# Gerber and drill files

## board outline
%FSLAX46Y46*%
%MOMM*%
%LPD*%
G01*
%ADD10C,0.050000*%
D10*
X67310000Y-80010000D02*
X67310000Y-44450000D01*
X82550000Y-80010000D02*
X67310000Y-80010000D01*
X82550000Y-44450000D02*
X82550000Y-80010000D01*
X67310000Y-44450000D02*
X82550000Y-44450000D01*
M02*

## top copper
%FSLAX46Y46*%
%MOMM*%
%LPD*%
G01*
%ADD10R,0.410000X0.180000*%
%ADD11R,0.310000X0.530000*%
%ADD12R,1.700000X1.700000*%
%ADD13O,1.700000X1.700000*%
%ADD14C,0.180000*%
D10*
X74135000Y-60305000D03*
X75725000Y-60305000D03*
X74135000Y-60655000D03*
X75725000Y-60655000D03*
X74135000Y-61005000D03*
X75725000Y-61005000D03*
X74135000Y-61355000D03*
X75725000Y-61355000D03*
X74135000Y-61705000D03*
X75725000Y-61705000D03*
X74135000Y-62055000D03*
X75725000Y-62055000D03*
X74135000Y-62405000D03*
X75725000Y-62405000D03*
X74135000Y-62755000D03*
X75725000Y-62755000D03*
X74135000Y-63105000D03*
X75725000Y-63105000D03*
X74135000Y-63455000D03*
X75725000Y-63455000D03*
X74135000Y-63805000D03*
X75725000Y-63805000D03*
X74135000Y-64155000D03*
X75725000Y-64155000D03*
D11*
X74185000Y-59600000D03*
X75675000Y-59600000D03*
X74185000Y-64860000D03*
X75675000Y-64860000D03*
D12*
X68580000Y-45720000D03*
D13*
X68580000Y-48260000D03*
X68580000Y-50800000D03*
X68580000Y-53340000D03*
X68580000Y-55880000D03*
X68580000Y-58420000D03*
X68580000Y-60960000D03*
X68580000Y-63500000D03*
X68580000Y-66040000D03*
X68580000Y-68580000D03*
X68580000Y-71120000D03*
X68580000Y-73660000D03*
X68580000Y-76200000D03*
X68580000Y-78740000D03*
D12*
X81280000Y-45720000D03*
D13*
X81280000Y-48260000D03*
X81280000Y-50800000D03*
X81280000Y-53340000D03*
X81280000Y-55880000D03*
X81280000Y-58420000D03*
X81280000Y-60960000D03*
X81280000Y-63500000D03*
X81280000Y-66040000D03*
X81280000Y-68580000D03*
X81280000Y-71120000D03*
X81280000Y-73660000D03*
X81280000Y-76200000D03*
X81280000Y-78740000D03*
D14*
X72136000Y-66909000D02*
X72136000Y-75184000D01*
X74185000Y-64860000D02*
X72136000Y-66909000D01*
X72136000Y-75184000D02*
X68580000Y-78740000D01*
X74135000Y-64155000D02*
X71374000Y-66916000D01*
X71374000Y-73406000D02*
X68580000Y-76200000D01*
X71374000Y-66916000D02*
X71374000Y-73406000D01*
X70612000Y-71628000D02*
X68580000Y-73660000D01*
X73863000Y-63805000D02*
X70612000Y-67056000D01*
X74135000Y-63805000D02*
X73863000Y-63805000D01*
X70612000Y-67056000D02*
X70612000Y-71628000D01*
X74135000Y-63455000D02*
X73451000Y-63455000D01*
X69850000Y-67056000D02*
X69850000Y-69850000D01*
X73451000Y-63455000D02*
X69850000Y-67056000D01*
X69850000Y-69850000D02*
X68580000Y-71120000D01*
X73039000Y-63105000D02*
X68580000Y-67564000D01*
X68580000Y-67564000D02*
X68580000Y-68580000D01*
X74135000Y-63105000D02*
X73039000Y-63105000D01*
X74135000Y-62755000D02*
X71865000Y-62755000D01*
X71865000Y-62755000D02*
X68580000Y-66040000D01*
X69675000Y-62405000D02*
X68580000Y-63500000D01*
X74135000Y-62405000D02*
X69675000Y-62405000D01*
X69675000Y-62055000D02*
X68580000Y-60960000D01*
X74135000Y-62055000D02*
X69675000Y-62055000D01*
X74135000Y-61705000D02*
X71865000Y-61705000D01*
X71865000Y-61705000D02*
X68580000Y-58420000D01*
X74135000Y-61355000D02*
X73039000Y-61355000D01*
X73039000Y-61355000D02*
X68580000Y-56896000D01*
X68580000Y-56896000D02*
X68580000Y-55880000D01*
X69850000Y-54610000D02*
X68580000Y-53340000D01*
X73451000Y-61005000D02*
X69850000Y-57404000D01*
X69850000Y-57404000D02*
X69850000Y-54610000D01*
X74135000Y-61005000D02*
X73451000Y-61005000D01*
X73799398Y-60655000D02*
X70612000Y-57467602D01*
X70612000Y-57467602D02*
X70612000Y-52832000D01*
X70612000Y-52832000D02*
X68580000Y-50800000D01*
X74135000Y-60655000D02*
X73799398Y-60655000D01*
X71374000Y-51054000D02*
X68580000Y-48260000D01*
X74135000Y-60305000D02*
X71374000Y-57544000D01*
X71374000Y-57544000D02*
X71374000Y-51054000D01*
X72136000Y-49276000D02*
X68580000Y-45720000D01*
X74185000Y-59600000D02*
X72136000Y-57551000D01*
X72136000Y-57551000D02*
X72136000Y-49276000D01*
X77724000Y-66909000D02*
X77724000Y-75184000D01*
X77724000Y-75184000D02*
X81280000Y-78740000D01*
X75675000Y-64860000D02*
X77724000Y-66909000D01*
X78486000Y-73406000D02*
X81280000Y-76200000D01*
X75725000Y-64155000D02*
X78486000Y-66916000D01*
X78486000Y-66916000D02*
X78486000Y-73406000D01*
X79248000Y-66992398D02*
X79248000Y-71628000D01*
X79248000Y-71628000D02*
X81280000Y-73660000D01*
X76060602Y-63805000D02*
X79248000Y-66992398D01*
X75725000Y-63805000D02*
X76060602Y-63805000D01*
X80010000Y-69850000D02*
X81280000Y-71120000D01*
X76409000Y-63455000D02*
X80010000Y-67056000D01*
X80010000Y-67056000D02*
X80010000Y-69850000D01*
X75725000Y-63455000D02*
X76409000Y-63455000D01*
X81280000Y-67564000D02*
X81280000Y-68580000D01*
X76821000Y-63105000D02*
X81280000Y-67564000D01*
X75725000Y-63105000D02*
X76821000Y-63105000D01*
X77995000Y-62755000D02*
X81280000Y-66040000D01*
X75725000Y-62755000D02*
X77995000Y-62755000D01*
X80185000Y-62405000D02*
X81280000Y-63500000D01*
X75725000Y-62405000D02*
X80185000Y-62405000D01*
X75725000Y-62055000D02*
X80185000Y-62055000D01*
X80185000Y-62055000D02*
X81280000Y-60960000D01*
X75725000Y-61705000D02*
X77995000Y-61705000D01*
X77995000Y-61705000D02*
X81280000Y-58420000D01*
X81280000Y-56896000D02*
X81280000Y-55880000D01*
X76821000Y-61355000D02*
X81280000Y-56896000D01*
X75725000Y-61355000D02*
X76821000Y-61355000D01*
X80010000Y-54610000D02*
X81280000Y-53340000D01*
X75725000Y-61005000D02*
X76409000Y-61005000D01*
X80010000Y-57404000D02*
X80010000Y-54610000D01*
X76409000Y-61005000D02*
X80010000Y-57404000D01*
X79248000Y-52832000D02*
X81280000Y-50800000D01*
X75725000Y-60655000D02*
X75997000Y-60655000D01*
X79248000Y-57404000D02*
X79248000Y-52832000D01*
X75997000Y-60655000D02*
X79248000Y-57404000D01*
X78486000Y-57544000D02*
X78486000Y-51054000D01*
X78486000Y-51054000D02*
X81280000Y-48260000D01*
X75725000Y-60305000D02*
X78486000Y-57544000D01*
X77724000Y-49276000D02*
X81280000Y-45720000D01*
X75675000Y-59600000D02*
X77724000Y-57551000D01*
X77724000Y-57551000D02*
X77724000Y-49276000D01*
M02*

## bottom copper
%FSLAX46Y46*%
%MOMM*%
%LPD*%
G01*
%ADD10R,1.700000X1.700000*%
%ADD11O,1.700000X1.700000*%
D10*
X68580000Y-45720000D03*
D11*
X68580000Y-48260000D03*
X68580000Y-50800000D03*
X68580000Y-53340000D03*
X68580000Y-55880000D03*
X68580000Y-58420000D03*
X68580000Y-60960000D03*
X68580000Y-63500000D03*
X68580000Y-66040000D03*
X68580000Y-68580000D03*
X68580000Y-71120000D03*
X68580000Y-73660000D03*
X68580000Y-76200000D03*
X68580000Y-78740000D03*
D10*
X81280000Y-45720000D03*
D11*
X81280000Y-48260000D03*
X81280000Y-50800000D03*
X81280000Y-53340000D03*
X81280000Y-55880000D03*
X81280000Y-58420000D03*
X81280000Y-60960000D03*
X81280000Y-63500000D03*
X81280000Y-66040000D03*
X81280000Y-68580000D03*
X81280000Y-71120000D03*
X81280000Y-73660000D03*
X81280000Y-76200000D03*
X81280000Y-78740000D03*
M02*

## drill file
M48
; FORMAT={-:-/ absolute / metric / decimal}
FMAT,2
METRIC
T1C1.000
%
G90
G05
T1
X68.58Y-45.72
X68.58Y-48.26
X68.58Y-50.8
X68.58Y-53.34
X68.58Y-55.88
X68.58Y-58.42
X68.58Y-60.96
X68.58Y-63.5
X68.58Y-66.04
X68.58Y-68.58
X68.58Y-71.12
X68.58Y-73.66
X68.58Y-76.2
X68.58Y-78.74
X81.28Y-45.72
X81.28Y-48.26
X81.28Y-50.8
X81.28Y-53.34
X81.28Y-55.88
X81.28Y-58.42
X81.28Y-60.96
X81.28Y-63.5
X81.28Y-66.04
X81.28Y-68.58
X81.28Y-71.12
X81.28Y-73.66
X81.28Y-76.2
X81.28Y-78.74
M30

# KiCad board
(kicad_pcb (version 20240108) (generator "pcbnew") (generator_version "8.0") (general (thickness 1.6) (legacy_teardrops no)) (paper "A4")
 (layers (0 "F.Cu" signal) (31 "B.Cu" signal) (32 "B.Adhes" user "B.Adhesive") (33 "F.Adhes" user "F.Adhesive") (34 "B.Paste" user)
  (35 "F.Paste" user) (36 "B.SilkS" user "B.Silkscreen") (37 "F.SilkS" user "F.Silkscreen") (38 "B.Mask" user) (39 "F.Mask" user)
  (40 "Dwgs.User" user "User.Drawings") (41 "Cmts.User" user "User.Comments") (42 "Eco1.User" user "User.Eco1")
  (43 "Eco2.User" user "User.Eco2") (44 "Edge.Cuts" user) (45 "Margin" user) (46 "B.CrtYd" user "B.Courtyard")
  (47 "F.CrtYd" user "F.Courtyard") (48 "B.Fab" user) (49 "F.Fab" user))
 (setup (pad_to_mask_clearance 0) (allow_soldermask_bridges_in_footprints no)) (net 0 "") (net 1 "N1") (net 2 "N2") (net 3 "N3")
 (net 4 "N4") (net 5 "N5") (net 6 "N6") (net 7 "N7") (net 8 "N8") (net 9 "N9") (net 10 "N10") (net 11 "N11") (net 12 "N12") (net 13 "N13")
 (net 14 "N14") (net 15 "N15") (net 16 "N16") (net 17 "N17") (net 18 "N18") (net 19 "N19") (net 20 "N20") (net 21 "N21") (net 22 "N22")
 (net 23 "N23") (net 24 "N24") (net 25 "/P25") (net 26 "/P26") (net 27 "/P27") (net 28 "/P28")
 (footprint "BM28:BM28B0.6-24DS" (layer "F.Cu") (at 74.93 62.23)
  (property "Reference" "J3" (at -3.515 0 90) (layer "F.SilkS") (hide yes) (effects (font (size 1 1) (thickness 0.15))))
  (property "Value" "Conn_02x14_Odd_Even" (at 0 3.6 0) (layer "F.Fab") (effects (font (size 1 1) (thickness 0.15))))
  (pad "1" smd rect (at -0.795 -1.925) (size 0.41 0.18) (layers "F.Cu" "F.Paste" "F.Mask") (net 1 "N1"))
  (pad "2" smd rect (at 0.795 -1.925) (size 0.41 0.18) (layers "F.Cu" "F.Paste" "F.Mask") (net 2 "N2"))
  (pad "3" smd rect (at -0.795 -1.575) (size 0.41 0.18) (layers "F.Cu" "F.Paste" "F.Mask") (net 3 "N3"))
  (pad "4" smd rect (at 0.795 -1.575) (size 0.41 0.18) (layers "F.Cu" "F.Paste" "F.Mask") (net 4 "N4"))
  (pad "5" smd rect (at -0.795 -1.225) (size 0.41 0.18) (layers "F.Cu" "F.Paste" "F.Mask") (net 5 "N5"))
  (pad "6" smd rect (at 0.795 -1.225) (size 0.41 0.18) (layers "F.Cu" "F.Paste" "F.Mask") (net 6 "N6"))
  (pad "7" smd rect (at -0.795 -0.875) (size 0.41 0.18) (layers "F.Cu" "F.Paste" "F.Mask") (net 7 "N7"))
  (pad "8" smd rect (at 0.795 -0.875) (size 0.41 0.18) (layers "F.Cu" "F.Paste" "F.Mask") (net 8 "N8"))
  (pad "9" smd rect (at -0.795 -0.525) (size 0.41 0.18) (layers "F.Cu" "F.Paste" "F.Mask") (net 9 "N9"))
  (pad "10" smd rect (at 0.795 -0.525) (size 0.41 0.18) (layers "F.Cu" "F.Paste" "F.Mask") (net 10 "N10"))
  (pad "11" smd rect (at -0.795 -0.175) (size 0.41 0.18) (layers "F.Cu" "F.Paste" "F.Mask") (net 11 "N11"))
  (pad "12" smd rect (at 0.795 -0.175) (size 0.41 0.18) (layers "F.Cu" "F.Paste" "F.Mask") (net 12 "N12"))
  (pad "13" smd rect (at -0.795 0.175) (size 0.41 0.18) (layers "F.Cu" "F.Paste" "F.Mask") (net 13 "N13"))
  (pad "14" smd rect (at 0.795 0.175) (size 0.41 0.18) (layers "F.Cu" "F.Paste" "F.Mask") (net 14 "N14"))
  (pad "15" smd rect (at -0.795 0.525) (size 0.41 0.18) (layers "F.Cu" "F.Paste" "F.Mask") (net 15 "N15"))
  (pad "16" smd rect (at 0.795 0.525) (size 0.41 0.18) (layers "F.Cu" "F.Paste" "F.Mask") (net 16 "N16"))
  (pad "17" smd rect (at -0.795 0.875) (size 0.41 0.18) (layers "F.Cu" "F.Paste" "F.Mask") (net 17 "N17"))
  (pad "18" smd rect (at 0.795 0.875) (size 0.41 0.18) (layers "F.Cu" "F.Paste" "F.Mask") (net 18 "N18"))
  (pad "19" smd rect (at -0.795 1.225) (size 0.41 0.18) (layers "F.Cu" "F.Paste" "F.Mask") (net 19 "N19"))
  (pad "20" smd rect (at 0.795 1.225) (size 0.41 0.18) (layers "F.Cu" "F.Paste" "F.Mask") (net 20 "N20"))
  (pad "21" smd rect (at -0.795 1.575) (size 0.41 0.18) (layers "F.Cu" "F.Paste" "F.Mask") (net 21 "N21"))
  (pad "22" smd rect (at 0.795 1.575) (size 0.41 0.18) (layers "F.Cu" "F.Paste" "F.Mask") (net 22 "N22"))
  (pad "23" smd rect (at -0.795 1.925) (size 0.41 0.18) (layers "F.Cu" "F.Paste" "F.Mask") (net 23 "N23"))
  (pad "24" smd rect (at 0.795 1.925) (size 0.41 0.18) (layers "F.Cu" "F.Paste" "F.Mask") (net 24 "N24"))
  (pad "25" smd rect (at -0.745 -2.63) (size 0.31 0.53) (layers "F.Cu" "F.Paste" "F.Mask") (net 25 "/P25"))
  (pad "26" smd rect (at 0.745 -2.63) (size 0.31 0.53) (layers "F.Cu" "F.Paste" "F.Mask") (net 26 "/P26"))
  (pad "27" smd rect (at -0.745 2.63) (size 0.31 0.53) (layers "F.Cu" "F.Paste" "F.Mask") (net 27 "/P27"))
  (pad "28" smd rect (at 0.745 2.63) (size 0.31 0.53) (layers "F.Cu" "F.Paste" "F.Mask") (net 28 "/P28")))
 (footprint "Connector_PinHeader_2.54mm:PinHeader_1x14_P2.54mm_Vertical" (layer "B.Cu") (at 68.58 45.72 180)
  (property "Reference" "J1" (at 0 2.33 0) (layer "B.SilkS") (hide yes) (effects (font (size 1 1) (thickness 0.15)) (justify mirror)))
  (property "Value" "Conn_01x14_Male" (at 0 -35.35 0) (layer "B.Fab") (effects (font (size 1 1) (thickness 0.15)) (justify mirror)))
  (pad "1" thru_hole rect (at 0 0 180) (size 1.7 1.7) (drill 1) (layers "*.Cu" "*.Mask") (remove_unused_layers no) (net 25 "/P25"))
  (pad "2" thru_hole oval (at 0 -2.54 180) (size 1.7 1.7) (drill 1) (layers "*.Cu" "*.Mask") (remove_unused_layers no) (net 1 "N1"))
  (pad "3" thru_hole oval (at 0 -5.08 180) (size 1.7 1.7) (drill 1) (layers "*.Cu" "*.Mask") (remove_unused_layers no) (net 3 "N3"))
  (pad "4" thru_hole oval (at 0 -7.62 180) (size 1.7 1.7) (drill 1) (layers "*.Cu" "*.Mask") (remove_unused_layers no) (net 5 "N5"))
  (pad "5" thru_hole oval (at 0 -10.16 180) (size 1.7 1.7) (drill 1) (layers "*.Cu" "*.Mask") (remove_unused_layers no) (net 7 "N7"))
  (pad "6" thru_hole oval (at 0 -12.7 180) (size 1.7 1.7) (drill 1) (layers "*.Cu" "*.Mask") (remove_unused_layers no) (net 9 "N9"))
  (pad "7" thru_hole oval (at 0 -15.24 180) (size 1.7 1.7) (drill 1) (layers "*.Cu" "*.Mask") (remove_unused_layers no) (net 11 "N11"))
  (pad "8" thru_hole oval (at 0 -17.78 180) (size 1.7 1.7) (drill 1) (layers "*.Cu" "*.Mask") (remove_unused_layers no) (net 13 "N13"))
  (pad "9" thru_hole oval (at 0 -20.32 180) (size 1.7 1.7) (drill 1) (layers "*.Cu" "*.Mask") (remove_unused_layers no) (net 15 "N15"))
  (pad "10" thru_hole oval (at 0 -22.86 180) (size 1.7 1.7) (drill 1) (layers "*.Cu" "*.Mask") (remove_unused_layers no) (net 17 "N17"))
  (pad "11" thru_hole oval (at 0 -25.4 180) (size 1.7 1.7) (drill 1) (layers "*.Cu" "*.Mask") (remove_unused_layers no) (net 19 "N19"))
  (pad "12" thru_hole oval (at 0 -27.94 180) (size 1.7 1.7) (drill 1) (layers "*.Cu" "*.Mask") (remove_unused_layers no) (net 21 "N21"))
  (pad "13" thru_hole oval (at 0 -30.48 180) (size 1.7 1.7) (drill 1) (layers "*.Cu" "*.Mask") (remove_unused_layers no) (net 23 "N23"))
  (pad "14" thru_hole oval (at 0 -33.02 180) (size 1.7 1.7) (drill 1) (layers "*.Cu" "*.Mask") (remove_unused_layers no) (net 27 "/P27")))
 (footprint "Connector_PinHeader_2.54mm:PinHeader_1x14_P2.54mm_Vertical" (layer "B.Cu") (at 81.28 45.72 180)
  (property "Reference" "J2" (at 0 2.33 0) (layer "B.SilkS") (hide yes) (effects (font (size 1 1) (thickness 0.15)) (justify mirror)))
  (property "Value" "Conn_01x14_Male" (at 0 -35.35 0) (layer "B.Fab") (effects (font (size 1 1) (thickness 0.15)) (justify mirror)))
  (pad "1" thru_hole rect (at 0 0 180) (size 1.7 1.7) (drill 1) (layers "*.Cu" "*.Mask") (remove_unused_layers no) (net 26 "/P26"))
  (pad "2" thru_hole oval (at 0 -2.54 180) (size 1.7 1.7) (drill 1) (layers "*.Cu" "*.Mask") (remove_unused_layers no) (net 2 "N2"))
  (pad "3" thru_hole oval (at 0 -5.08 180) (size 1.7 1.7) (drill 1) (layers "*.Cu" "*.Mask") (remove_unused_layers no) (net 4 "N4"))
  (pad "4" thru_hole oval (at 0 -7.62 180) (size 1.7 1.7) (drill 1) (layers "*.Cu" "*.Mask") (remove_unused_layers no) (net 6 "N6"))
  (pad "5" thru_hole oval (at 0 -10.16 180) (size 1.7 1.7) (drill 1) (layers "*.Cu" "*.Mask") (remove_unused_layers no) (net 8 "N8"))
  (pad "6" thru_hole oval (at 0 -12.7 180) (size 1.7 1.7) (drill 1) (layers "*.Cu" "*.Mask") (remove_unused_layers no) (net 10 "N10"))
  (pad "7" thru_hole oval (at 0 -15.24 180) (size 1.7 1.7) (drill 1) (layers "*.Cu" "*.Mask") (remove_unused_layers no) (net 12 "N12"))
  (pad "8" thru_hole oval (at 0 -17.78 180) (size 1.7 1.7) (drill 1) (layers "*.Cu" "*.Mask") (remove_unused_layers no) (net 14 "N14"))
  (pad "9" thru_hole oval (at 0 -20.32 180) (size 1.7 1.7) (drill 1) (layers "*.Cu" "*.Mask") (remove_unused_layers no) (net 16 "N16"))
  (pad "10" thru_hole oval (at 0 -22.86 180) (size 1.7 1.7) (drill 1) (layers "*.Cu" "*.Mask") (remove_unused_layers no) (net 18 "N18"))
  (pad "11" thru_hole oval (at 0 -25.4 180) (size 1.7 1.7) (drill 1) (layers "*.Cu" "*.Mask") (remove_unused_layers no) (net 20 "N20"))
  (pad "12" thru_hole oval (at 0 -27.94 180) (size 1.7 1.7) (drill 1) (layers "*.Cu" "*.Mask") (remove_unused_layers no) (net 22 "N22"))
  (pad "13" thru_hole oval (at 0 -30.48 180) (size 1.7 1.7) (drill 1) (layers "*.Cu" "*.Mask") (remove_unused_layers no) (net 24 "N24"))
  (pad "14" thru_hole oval (at 0 -33.02 180) (size 1.7 1.7) (drill 1) (layers "*.Cu" "*.Mask") (remove_unused_layers no) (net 28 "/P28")))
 (gr_line (start 67.31 80.01) (end 67.31 44.45) (stroke (width 0.05) (type solid)) (layer "Edge.Cuts"))
 (gr_line (start 82.55 80.01) (end 67.31 80.01) (stroke (width 0.05) (type solid)) (layer "Edge.Cuts"))
 (gr_line (start 82.55 44.45) (end 82.55 80.01) (stroke (width 0.05) (type solid)) (layer "Edge.Cuts"))
 (gr_line (start 67.31 44.45) (end 82.55 44.45) (stroke (width 0.05) (type solid)) (layer "Edge.Cuts"))
 (segment (start 72.136 66.909) (end 72.136 75.184) (width 0.18) (layer "F.Cu") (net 27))
 (segment (start 74.185 64.86) (end 72.136 66.909) (width 0.18) (layer "F.Cu") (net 27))
 (segment (start 72.136 75.184) (end 68.58 78.74) (width 0.18) (layer "F.Cu") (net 27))
 (segment (start 74.135 64.155) (end 71.374 66.916) (width 0.18) (layer "F.Cu") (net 23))
 (segment (start 71.374 73.406) (end 68.58 76.2) (width 0.18) (layer "F.Cu") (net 23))
 (segment (start 71.374 66.916) (end 71.374 73.406) (width 0.18) (layer "F.Cu") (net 23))
 (segment (start 70.612 71.628) (end 68.58 73.66) (width 0.18) (layer "F.Cu") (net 21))
 (segment (start 73.863 63.805) (end 70.612 67.056) (width 0.18) (layer "F.Cu") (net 21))
 (segment (start 74.135 63.805) (end 73.863 63.805) (width 0.18) (layer "F.Cu") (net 21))
 (segment (start 70.612 67.056) (end 70.612 71.628) (width 0.18) (layer "F.Cu") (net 21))
 (segment (start 74.135 63.455) (end 73.451 63.455) (width 0.18) (layer "F.Cu") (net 19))
 (segment (start 69.85 67.056) (end 69.85 69.85) (width 0.18) (layer "F.Cu") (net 19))
 (segment (start 73.451 63.455) (end 69.85 67.056) (width 0.18) (layer "F.Cu") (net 19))
 (segment (start 69.85 69.85) (end 68.58 71.12) (width 0.18) (layer "F.Cu") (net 19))
 (segment (start 73.039 63.105) (end 68.58 67.564) (width 0.18) (layer "F.Cu") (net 17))
 (segment (start 68.58 67.564) (end 68.58 68.58) (width 0.18) (layer "F.Cu") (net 17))
 (segment (start 74.135 63.105) (end 73.039 63.105) (width 0.18) (layer "F.Cu") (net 17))
 (segment (start 74.135 62.755) (end 71.865 62.755) (width 0.18) (layer "F.Cu") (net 15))
 (segment (start 71.865 62.755) (end 68.58 66.04) (width 0.18) (layer "F.Cu") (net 15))
 (segment (start 69.675 62.405) (end 68.58 63.5) (width 0.18) (layer "F.Cu") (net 13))
 (segment (start 74.135 62.405) (end 69.675 62.405) (width 0.18) (layer "F.Cu") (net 13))
 (segment (start 69.675 62.055) (end 68.58 60.96) (width 0.18) (layer "F.Cu") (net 11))
 (segment (start 74.135 62.055) (end 69.675 62.055) (width 0.18) (layer "F.Cu") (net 11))
 (segment (start 74.135 61.705) (end 71.865 61.705) (width 0.18) (layer "F.Cu") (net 9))
 (segment (start 71.865 61.705) (end 68.58 58.42) (width 0.18) (layer "F.Cu") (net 9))
 (segment (start 74.135 61.355) (end 73.039 61.355) (width 0.18) (layer "F.Cu") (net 7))
 (segment (start 73.039 61.355) (end 68.58 56.896) (width 0.18) (layer "F.Cu") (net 7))
 (segment (start 68.58 56.896) (end 68.58 55.88) (width 0.18) (layer "F.Cu") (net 7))
 (segment (start 69.85 54.61) (end 68.58 53.34) (width 0.18) (layer "F.Cu") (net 5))
 (segment (start 73.451 61.005) (end 69.85 57.404) (width 0.18) (layer "F.Cu") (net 5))
 (segment (start 69.85 57.404) (end 69.85 54.61) (width 0.18) (layer "F.Cu") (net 5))
 (segment (start 74.135 61.005) (end 73.451 61.005) (width 0.18) (layer "F.Cu") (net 5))
 (segment (start 73.799398 60.655) (end 70.612 57.467602) (width 0.18) (layer "F.Cu") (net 3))
 (segment (start 70.612 57.467602) (end 70.612 52.832) (width 0.18) (layer "F.Cu") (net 3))
 (segment (start 70.612 52.832) (end 68.58 50.8) (width 0.18) (layer "F.Cu") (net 3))
 (segment (start 74.135 60.655) (end 73.799398 60.655) (width 0.18) (layer "F.Cu") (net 3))
 (segment (start 71.374 51.054) (end 68.58 48.26) (width 0.18) (layer "F.Cu") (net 1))
 (segment (start 74.135 60.305) (end 71.374 57.544) (width 0.18) (layer "F.Cu") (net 1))
 (segment (start 71.374 57.544) (end 71.374 51.054) (width 0.18) (layer "F.Cu") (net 1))
 (segment (start 72.136 49.276) (end 68.58 45.72) (width 0.18) (layer "F.Cu") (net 25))
 (segment (start 74.185 59.6) (end 72.136 57.551) (width 0.18) (layer "F.Cu") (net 25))
 (segment (start 72.136 57.551) (end 72.136 49.276) (width 0.18) (layer "F.Cu") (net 25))
 (segment (start 77.724 66.909) (end 77.724 75.184) (width 0.18) (layer "F.Cu") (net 28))
 (segment (start 77.724 75.184) (end 81.28 78.74) (width 0.18) (layer "F.Cu") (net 28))
 (segment (start 75.675 64.86) (end 77.724 66.909) (width 0.18) (layer "F.Cu") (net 28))
 (segment (start 78.486 73.406) (end 81.28 76.2) (width 0.18) (layer "F.Cu") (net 24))
 (segment (start 75.725 64.155) (end 78.486 66.916) (width 0.18) (layer "F.Cu") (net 24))
 (segment (start 78.486 66.916) (end 78.486 73.406) (width 0.18) (layer "F.Cu") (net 24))
 (segment (start 79.248 66.992398) (end 79.248 71.628) (width 0.18) (layer "F.Cu") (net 22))
 (segment (start 79.248 71.628) (end 81.28 73.66) (width 0.18) (layer "F.Cu") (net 22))
 (segment (start 76.060602 63.805) (end 79.248 66.992398) (width 0.18) (layer "F.Cu") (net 22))
 (segment (start 75.725 63.805) (end 76.060602 63.805) (width 0.18) (layer "F.Cu") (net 22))
 (segment (start 80.01 69.85) (end 81.28 71.12) (width 0.18) (layer "F.Cu") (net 20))
 (segment (start 76.409 63.455) (end 80.01 67.056) (width 0.18) (layer "F.Cu") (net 20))
 (segment (start 80.01 67.056) (end 80.01 69.85) (width 0.18) (layer "F.Cu") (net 20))
 (segment (start 75.725 63.455) (end 76.409 63.455) (width 0.18) (layer "F.Cu") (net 20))
 (segment (start 81.28 67.564) (end 81.28 68.58) (width 0.18) (layer "F.Cu") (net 18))
 (segment (start 76.821 63.105) (end 81.28 67.564) (width 0.18) (layer "F.Cu") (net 18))
 (segment (start 75.725 63.105) (end 76.821 63.105) (width 0.18) (layer "F.Cu") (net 18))
 (segment (start 77.995 62.755) (end 81.28 66.04) (width 0.18) (layer "F.Cu") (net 16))
 (segment (start 75.725 62.755) (end 77.995 62.755) (width 0.18) (layer "F.Cu") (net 16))
 (segment (start 80.185 62.405) (end 81.28 63.5) (width 0.18) (layer "F.Cu") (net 14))
 (segment (start 75.725 62.405) (end 80.185 62.405) (width 0.18) (layer "F.Cu") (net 14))
 (segment (start 75.725 62.055) (end 80.185 62.055) (width 0.18) (layer "F.Cu") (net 12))
 (segment (start 80.185 62.055) (end 81.28 60.96) (width 0.18) (layer "F.Cu") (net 12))
 (segment (start 75.725 61.705) (end 77.995 61.705) (width 0.18) (layer "F.Cu") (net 10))
 (segment (start 77.995 61.705) (end 81.28 58.42) (width 0.18) (layer "F.Cu") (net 10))
 (segment (start 81.28 56.896) (end 81.28 55.88) (width 0.18) (layer "F.Cu") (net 8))
 (segment (start 76.821 61.355) (end 81.28 56.896) (width 0.18) (layer "F.Cu") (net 8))
 (segment (start 75.725 61.355) (end 76.821 61.355) (width 0.18) (layer "F.Cu") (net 8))
 (segment (start 80.01 54.61) (end 81.28 53.34) (width 0.18) (layer "F.Cu") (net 6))
 (segment (start 75.725 61.005) (end 76.409 61.005) (width 0.18) (layer "F.Cu") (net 6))
 (segment (start 80.01 57.404) (end 80.01 54.61) (width 0.18) (layer "F.Cu") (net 6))
 (segment (start 76.409 61.005) (end 80.01 57.404) (width 0.18) (layer "F.Cu") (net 6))
 (segment (start 79.248 52.832) (end 81.28 50.8) (width 0.18) (layer "F.Cu") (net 4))
 (segment (start 75.725 60.655) (end 75.997 60.655) (width 0.18) (layer "F.Cu") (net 4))
 (segment (start 79.248 57.404) (end 79.248 52.832) (width 0.18) (layer "F.Cu") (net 4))
 (segment (start 75.997 60.655) (end 79.248 57.404) (width 0.18) (layer "F.Cu") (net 4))
 (segment (start 78.486 57.544) (end 78.486 51.054) (width 0.18) (layer "F.Cu") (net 2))
 (segment (start 78.486 51.054) (end 81.28 48.26) (width 0.18) (layer "F.Cu") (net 2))
 (segment (start 75.725 60.305) (end 78.486 57.544) (width 0.18) (layer "F.Cu") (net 2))
 (segment (start 77.724 49.276) (end 81.28 45.72) (width 0.18) (layer "F.Cu") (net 26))
 (segment (start 75.675 59.6) (end 77.724 57.551) (width 0.18) (layer "F.Cu") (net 26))
 (segment (start 77.724 57.551) (end 77.724 49.276) (width 0.18) (layer "F.Cu") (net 26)))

